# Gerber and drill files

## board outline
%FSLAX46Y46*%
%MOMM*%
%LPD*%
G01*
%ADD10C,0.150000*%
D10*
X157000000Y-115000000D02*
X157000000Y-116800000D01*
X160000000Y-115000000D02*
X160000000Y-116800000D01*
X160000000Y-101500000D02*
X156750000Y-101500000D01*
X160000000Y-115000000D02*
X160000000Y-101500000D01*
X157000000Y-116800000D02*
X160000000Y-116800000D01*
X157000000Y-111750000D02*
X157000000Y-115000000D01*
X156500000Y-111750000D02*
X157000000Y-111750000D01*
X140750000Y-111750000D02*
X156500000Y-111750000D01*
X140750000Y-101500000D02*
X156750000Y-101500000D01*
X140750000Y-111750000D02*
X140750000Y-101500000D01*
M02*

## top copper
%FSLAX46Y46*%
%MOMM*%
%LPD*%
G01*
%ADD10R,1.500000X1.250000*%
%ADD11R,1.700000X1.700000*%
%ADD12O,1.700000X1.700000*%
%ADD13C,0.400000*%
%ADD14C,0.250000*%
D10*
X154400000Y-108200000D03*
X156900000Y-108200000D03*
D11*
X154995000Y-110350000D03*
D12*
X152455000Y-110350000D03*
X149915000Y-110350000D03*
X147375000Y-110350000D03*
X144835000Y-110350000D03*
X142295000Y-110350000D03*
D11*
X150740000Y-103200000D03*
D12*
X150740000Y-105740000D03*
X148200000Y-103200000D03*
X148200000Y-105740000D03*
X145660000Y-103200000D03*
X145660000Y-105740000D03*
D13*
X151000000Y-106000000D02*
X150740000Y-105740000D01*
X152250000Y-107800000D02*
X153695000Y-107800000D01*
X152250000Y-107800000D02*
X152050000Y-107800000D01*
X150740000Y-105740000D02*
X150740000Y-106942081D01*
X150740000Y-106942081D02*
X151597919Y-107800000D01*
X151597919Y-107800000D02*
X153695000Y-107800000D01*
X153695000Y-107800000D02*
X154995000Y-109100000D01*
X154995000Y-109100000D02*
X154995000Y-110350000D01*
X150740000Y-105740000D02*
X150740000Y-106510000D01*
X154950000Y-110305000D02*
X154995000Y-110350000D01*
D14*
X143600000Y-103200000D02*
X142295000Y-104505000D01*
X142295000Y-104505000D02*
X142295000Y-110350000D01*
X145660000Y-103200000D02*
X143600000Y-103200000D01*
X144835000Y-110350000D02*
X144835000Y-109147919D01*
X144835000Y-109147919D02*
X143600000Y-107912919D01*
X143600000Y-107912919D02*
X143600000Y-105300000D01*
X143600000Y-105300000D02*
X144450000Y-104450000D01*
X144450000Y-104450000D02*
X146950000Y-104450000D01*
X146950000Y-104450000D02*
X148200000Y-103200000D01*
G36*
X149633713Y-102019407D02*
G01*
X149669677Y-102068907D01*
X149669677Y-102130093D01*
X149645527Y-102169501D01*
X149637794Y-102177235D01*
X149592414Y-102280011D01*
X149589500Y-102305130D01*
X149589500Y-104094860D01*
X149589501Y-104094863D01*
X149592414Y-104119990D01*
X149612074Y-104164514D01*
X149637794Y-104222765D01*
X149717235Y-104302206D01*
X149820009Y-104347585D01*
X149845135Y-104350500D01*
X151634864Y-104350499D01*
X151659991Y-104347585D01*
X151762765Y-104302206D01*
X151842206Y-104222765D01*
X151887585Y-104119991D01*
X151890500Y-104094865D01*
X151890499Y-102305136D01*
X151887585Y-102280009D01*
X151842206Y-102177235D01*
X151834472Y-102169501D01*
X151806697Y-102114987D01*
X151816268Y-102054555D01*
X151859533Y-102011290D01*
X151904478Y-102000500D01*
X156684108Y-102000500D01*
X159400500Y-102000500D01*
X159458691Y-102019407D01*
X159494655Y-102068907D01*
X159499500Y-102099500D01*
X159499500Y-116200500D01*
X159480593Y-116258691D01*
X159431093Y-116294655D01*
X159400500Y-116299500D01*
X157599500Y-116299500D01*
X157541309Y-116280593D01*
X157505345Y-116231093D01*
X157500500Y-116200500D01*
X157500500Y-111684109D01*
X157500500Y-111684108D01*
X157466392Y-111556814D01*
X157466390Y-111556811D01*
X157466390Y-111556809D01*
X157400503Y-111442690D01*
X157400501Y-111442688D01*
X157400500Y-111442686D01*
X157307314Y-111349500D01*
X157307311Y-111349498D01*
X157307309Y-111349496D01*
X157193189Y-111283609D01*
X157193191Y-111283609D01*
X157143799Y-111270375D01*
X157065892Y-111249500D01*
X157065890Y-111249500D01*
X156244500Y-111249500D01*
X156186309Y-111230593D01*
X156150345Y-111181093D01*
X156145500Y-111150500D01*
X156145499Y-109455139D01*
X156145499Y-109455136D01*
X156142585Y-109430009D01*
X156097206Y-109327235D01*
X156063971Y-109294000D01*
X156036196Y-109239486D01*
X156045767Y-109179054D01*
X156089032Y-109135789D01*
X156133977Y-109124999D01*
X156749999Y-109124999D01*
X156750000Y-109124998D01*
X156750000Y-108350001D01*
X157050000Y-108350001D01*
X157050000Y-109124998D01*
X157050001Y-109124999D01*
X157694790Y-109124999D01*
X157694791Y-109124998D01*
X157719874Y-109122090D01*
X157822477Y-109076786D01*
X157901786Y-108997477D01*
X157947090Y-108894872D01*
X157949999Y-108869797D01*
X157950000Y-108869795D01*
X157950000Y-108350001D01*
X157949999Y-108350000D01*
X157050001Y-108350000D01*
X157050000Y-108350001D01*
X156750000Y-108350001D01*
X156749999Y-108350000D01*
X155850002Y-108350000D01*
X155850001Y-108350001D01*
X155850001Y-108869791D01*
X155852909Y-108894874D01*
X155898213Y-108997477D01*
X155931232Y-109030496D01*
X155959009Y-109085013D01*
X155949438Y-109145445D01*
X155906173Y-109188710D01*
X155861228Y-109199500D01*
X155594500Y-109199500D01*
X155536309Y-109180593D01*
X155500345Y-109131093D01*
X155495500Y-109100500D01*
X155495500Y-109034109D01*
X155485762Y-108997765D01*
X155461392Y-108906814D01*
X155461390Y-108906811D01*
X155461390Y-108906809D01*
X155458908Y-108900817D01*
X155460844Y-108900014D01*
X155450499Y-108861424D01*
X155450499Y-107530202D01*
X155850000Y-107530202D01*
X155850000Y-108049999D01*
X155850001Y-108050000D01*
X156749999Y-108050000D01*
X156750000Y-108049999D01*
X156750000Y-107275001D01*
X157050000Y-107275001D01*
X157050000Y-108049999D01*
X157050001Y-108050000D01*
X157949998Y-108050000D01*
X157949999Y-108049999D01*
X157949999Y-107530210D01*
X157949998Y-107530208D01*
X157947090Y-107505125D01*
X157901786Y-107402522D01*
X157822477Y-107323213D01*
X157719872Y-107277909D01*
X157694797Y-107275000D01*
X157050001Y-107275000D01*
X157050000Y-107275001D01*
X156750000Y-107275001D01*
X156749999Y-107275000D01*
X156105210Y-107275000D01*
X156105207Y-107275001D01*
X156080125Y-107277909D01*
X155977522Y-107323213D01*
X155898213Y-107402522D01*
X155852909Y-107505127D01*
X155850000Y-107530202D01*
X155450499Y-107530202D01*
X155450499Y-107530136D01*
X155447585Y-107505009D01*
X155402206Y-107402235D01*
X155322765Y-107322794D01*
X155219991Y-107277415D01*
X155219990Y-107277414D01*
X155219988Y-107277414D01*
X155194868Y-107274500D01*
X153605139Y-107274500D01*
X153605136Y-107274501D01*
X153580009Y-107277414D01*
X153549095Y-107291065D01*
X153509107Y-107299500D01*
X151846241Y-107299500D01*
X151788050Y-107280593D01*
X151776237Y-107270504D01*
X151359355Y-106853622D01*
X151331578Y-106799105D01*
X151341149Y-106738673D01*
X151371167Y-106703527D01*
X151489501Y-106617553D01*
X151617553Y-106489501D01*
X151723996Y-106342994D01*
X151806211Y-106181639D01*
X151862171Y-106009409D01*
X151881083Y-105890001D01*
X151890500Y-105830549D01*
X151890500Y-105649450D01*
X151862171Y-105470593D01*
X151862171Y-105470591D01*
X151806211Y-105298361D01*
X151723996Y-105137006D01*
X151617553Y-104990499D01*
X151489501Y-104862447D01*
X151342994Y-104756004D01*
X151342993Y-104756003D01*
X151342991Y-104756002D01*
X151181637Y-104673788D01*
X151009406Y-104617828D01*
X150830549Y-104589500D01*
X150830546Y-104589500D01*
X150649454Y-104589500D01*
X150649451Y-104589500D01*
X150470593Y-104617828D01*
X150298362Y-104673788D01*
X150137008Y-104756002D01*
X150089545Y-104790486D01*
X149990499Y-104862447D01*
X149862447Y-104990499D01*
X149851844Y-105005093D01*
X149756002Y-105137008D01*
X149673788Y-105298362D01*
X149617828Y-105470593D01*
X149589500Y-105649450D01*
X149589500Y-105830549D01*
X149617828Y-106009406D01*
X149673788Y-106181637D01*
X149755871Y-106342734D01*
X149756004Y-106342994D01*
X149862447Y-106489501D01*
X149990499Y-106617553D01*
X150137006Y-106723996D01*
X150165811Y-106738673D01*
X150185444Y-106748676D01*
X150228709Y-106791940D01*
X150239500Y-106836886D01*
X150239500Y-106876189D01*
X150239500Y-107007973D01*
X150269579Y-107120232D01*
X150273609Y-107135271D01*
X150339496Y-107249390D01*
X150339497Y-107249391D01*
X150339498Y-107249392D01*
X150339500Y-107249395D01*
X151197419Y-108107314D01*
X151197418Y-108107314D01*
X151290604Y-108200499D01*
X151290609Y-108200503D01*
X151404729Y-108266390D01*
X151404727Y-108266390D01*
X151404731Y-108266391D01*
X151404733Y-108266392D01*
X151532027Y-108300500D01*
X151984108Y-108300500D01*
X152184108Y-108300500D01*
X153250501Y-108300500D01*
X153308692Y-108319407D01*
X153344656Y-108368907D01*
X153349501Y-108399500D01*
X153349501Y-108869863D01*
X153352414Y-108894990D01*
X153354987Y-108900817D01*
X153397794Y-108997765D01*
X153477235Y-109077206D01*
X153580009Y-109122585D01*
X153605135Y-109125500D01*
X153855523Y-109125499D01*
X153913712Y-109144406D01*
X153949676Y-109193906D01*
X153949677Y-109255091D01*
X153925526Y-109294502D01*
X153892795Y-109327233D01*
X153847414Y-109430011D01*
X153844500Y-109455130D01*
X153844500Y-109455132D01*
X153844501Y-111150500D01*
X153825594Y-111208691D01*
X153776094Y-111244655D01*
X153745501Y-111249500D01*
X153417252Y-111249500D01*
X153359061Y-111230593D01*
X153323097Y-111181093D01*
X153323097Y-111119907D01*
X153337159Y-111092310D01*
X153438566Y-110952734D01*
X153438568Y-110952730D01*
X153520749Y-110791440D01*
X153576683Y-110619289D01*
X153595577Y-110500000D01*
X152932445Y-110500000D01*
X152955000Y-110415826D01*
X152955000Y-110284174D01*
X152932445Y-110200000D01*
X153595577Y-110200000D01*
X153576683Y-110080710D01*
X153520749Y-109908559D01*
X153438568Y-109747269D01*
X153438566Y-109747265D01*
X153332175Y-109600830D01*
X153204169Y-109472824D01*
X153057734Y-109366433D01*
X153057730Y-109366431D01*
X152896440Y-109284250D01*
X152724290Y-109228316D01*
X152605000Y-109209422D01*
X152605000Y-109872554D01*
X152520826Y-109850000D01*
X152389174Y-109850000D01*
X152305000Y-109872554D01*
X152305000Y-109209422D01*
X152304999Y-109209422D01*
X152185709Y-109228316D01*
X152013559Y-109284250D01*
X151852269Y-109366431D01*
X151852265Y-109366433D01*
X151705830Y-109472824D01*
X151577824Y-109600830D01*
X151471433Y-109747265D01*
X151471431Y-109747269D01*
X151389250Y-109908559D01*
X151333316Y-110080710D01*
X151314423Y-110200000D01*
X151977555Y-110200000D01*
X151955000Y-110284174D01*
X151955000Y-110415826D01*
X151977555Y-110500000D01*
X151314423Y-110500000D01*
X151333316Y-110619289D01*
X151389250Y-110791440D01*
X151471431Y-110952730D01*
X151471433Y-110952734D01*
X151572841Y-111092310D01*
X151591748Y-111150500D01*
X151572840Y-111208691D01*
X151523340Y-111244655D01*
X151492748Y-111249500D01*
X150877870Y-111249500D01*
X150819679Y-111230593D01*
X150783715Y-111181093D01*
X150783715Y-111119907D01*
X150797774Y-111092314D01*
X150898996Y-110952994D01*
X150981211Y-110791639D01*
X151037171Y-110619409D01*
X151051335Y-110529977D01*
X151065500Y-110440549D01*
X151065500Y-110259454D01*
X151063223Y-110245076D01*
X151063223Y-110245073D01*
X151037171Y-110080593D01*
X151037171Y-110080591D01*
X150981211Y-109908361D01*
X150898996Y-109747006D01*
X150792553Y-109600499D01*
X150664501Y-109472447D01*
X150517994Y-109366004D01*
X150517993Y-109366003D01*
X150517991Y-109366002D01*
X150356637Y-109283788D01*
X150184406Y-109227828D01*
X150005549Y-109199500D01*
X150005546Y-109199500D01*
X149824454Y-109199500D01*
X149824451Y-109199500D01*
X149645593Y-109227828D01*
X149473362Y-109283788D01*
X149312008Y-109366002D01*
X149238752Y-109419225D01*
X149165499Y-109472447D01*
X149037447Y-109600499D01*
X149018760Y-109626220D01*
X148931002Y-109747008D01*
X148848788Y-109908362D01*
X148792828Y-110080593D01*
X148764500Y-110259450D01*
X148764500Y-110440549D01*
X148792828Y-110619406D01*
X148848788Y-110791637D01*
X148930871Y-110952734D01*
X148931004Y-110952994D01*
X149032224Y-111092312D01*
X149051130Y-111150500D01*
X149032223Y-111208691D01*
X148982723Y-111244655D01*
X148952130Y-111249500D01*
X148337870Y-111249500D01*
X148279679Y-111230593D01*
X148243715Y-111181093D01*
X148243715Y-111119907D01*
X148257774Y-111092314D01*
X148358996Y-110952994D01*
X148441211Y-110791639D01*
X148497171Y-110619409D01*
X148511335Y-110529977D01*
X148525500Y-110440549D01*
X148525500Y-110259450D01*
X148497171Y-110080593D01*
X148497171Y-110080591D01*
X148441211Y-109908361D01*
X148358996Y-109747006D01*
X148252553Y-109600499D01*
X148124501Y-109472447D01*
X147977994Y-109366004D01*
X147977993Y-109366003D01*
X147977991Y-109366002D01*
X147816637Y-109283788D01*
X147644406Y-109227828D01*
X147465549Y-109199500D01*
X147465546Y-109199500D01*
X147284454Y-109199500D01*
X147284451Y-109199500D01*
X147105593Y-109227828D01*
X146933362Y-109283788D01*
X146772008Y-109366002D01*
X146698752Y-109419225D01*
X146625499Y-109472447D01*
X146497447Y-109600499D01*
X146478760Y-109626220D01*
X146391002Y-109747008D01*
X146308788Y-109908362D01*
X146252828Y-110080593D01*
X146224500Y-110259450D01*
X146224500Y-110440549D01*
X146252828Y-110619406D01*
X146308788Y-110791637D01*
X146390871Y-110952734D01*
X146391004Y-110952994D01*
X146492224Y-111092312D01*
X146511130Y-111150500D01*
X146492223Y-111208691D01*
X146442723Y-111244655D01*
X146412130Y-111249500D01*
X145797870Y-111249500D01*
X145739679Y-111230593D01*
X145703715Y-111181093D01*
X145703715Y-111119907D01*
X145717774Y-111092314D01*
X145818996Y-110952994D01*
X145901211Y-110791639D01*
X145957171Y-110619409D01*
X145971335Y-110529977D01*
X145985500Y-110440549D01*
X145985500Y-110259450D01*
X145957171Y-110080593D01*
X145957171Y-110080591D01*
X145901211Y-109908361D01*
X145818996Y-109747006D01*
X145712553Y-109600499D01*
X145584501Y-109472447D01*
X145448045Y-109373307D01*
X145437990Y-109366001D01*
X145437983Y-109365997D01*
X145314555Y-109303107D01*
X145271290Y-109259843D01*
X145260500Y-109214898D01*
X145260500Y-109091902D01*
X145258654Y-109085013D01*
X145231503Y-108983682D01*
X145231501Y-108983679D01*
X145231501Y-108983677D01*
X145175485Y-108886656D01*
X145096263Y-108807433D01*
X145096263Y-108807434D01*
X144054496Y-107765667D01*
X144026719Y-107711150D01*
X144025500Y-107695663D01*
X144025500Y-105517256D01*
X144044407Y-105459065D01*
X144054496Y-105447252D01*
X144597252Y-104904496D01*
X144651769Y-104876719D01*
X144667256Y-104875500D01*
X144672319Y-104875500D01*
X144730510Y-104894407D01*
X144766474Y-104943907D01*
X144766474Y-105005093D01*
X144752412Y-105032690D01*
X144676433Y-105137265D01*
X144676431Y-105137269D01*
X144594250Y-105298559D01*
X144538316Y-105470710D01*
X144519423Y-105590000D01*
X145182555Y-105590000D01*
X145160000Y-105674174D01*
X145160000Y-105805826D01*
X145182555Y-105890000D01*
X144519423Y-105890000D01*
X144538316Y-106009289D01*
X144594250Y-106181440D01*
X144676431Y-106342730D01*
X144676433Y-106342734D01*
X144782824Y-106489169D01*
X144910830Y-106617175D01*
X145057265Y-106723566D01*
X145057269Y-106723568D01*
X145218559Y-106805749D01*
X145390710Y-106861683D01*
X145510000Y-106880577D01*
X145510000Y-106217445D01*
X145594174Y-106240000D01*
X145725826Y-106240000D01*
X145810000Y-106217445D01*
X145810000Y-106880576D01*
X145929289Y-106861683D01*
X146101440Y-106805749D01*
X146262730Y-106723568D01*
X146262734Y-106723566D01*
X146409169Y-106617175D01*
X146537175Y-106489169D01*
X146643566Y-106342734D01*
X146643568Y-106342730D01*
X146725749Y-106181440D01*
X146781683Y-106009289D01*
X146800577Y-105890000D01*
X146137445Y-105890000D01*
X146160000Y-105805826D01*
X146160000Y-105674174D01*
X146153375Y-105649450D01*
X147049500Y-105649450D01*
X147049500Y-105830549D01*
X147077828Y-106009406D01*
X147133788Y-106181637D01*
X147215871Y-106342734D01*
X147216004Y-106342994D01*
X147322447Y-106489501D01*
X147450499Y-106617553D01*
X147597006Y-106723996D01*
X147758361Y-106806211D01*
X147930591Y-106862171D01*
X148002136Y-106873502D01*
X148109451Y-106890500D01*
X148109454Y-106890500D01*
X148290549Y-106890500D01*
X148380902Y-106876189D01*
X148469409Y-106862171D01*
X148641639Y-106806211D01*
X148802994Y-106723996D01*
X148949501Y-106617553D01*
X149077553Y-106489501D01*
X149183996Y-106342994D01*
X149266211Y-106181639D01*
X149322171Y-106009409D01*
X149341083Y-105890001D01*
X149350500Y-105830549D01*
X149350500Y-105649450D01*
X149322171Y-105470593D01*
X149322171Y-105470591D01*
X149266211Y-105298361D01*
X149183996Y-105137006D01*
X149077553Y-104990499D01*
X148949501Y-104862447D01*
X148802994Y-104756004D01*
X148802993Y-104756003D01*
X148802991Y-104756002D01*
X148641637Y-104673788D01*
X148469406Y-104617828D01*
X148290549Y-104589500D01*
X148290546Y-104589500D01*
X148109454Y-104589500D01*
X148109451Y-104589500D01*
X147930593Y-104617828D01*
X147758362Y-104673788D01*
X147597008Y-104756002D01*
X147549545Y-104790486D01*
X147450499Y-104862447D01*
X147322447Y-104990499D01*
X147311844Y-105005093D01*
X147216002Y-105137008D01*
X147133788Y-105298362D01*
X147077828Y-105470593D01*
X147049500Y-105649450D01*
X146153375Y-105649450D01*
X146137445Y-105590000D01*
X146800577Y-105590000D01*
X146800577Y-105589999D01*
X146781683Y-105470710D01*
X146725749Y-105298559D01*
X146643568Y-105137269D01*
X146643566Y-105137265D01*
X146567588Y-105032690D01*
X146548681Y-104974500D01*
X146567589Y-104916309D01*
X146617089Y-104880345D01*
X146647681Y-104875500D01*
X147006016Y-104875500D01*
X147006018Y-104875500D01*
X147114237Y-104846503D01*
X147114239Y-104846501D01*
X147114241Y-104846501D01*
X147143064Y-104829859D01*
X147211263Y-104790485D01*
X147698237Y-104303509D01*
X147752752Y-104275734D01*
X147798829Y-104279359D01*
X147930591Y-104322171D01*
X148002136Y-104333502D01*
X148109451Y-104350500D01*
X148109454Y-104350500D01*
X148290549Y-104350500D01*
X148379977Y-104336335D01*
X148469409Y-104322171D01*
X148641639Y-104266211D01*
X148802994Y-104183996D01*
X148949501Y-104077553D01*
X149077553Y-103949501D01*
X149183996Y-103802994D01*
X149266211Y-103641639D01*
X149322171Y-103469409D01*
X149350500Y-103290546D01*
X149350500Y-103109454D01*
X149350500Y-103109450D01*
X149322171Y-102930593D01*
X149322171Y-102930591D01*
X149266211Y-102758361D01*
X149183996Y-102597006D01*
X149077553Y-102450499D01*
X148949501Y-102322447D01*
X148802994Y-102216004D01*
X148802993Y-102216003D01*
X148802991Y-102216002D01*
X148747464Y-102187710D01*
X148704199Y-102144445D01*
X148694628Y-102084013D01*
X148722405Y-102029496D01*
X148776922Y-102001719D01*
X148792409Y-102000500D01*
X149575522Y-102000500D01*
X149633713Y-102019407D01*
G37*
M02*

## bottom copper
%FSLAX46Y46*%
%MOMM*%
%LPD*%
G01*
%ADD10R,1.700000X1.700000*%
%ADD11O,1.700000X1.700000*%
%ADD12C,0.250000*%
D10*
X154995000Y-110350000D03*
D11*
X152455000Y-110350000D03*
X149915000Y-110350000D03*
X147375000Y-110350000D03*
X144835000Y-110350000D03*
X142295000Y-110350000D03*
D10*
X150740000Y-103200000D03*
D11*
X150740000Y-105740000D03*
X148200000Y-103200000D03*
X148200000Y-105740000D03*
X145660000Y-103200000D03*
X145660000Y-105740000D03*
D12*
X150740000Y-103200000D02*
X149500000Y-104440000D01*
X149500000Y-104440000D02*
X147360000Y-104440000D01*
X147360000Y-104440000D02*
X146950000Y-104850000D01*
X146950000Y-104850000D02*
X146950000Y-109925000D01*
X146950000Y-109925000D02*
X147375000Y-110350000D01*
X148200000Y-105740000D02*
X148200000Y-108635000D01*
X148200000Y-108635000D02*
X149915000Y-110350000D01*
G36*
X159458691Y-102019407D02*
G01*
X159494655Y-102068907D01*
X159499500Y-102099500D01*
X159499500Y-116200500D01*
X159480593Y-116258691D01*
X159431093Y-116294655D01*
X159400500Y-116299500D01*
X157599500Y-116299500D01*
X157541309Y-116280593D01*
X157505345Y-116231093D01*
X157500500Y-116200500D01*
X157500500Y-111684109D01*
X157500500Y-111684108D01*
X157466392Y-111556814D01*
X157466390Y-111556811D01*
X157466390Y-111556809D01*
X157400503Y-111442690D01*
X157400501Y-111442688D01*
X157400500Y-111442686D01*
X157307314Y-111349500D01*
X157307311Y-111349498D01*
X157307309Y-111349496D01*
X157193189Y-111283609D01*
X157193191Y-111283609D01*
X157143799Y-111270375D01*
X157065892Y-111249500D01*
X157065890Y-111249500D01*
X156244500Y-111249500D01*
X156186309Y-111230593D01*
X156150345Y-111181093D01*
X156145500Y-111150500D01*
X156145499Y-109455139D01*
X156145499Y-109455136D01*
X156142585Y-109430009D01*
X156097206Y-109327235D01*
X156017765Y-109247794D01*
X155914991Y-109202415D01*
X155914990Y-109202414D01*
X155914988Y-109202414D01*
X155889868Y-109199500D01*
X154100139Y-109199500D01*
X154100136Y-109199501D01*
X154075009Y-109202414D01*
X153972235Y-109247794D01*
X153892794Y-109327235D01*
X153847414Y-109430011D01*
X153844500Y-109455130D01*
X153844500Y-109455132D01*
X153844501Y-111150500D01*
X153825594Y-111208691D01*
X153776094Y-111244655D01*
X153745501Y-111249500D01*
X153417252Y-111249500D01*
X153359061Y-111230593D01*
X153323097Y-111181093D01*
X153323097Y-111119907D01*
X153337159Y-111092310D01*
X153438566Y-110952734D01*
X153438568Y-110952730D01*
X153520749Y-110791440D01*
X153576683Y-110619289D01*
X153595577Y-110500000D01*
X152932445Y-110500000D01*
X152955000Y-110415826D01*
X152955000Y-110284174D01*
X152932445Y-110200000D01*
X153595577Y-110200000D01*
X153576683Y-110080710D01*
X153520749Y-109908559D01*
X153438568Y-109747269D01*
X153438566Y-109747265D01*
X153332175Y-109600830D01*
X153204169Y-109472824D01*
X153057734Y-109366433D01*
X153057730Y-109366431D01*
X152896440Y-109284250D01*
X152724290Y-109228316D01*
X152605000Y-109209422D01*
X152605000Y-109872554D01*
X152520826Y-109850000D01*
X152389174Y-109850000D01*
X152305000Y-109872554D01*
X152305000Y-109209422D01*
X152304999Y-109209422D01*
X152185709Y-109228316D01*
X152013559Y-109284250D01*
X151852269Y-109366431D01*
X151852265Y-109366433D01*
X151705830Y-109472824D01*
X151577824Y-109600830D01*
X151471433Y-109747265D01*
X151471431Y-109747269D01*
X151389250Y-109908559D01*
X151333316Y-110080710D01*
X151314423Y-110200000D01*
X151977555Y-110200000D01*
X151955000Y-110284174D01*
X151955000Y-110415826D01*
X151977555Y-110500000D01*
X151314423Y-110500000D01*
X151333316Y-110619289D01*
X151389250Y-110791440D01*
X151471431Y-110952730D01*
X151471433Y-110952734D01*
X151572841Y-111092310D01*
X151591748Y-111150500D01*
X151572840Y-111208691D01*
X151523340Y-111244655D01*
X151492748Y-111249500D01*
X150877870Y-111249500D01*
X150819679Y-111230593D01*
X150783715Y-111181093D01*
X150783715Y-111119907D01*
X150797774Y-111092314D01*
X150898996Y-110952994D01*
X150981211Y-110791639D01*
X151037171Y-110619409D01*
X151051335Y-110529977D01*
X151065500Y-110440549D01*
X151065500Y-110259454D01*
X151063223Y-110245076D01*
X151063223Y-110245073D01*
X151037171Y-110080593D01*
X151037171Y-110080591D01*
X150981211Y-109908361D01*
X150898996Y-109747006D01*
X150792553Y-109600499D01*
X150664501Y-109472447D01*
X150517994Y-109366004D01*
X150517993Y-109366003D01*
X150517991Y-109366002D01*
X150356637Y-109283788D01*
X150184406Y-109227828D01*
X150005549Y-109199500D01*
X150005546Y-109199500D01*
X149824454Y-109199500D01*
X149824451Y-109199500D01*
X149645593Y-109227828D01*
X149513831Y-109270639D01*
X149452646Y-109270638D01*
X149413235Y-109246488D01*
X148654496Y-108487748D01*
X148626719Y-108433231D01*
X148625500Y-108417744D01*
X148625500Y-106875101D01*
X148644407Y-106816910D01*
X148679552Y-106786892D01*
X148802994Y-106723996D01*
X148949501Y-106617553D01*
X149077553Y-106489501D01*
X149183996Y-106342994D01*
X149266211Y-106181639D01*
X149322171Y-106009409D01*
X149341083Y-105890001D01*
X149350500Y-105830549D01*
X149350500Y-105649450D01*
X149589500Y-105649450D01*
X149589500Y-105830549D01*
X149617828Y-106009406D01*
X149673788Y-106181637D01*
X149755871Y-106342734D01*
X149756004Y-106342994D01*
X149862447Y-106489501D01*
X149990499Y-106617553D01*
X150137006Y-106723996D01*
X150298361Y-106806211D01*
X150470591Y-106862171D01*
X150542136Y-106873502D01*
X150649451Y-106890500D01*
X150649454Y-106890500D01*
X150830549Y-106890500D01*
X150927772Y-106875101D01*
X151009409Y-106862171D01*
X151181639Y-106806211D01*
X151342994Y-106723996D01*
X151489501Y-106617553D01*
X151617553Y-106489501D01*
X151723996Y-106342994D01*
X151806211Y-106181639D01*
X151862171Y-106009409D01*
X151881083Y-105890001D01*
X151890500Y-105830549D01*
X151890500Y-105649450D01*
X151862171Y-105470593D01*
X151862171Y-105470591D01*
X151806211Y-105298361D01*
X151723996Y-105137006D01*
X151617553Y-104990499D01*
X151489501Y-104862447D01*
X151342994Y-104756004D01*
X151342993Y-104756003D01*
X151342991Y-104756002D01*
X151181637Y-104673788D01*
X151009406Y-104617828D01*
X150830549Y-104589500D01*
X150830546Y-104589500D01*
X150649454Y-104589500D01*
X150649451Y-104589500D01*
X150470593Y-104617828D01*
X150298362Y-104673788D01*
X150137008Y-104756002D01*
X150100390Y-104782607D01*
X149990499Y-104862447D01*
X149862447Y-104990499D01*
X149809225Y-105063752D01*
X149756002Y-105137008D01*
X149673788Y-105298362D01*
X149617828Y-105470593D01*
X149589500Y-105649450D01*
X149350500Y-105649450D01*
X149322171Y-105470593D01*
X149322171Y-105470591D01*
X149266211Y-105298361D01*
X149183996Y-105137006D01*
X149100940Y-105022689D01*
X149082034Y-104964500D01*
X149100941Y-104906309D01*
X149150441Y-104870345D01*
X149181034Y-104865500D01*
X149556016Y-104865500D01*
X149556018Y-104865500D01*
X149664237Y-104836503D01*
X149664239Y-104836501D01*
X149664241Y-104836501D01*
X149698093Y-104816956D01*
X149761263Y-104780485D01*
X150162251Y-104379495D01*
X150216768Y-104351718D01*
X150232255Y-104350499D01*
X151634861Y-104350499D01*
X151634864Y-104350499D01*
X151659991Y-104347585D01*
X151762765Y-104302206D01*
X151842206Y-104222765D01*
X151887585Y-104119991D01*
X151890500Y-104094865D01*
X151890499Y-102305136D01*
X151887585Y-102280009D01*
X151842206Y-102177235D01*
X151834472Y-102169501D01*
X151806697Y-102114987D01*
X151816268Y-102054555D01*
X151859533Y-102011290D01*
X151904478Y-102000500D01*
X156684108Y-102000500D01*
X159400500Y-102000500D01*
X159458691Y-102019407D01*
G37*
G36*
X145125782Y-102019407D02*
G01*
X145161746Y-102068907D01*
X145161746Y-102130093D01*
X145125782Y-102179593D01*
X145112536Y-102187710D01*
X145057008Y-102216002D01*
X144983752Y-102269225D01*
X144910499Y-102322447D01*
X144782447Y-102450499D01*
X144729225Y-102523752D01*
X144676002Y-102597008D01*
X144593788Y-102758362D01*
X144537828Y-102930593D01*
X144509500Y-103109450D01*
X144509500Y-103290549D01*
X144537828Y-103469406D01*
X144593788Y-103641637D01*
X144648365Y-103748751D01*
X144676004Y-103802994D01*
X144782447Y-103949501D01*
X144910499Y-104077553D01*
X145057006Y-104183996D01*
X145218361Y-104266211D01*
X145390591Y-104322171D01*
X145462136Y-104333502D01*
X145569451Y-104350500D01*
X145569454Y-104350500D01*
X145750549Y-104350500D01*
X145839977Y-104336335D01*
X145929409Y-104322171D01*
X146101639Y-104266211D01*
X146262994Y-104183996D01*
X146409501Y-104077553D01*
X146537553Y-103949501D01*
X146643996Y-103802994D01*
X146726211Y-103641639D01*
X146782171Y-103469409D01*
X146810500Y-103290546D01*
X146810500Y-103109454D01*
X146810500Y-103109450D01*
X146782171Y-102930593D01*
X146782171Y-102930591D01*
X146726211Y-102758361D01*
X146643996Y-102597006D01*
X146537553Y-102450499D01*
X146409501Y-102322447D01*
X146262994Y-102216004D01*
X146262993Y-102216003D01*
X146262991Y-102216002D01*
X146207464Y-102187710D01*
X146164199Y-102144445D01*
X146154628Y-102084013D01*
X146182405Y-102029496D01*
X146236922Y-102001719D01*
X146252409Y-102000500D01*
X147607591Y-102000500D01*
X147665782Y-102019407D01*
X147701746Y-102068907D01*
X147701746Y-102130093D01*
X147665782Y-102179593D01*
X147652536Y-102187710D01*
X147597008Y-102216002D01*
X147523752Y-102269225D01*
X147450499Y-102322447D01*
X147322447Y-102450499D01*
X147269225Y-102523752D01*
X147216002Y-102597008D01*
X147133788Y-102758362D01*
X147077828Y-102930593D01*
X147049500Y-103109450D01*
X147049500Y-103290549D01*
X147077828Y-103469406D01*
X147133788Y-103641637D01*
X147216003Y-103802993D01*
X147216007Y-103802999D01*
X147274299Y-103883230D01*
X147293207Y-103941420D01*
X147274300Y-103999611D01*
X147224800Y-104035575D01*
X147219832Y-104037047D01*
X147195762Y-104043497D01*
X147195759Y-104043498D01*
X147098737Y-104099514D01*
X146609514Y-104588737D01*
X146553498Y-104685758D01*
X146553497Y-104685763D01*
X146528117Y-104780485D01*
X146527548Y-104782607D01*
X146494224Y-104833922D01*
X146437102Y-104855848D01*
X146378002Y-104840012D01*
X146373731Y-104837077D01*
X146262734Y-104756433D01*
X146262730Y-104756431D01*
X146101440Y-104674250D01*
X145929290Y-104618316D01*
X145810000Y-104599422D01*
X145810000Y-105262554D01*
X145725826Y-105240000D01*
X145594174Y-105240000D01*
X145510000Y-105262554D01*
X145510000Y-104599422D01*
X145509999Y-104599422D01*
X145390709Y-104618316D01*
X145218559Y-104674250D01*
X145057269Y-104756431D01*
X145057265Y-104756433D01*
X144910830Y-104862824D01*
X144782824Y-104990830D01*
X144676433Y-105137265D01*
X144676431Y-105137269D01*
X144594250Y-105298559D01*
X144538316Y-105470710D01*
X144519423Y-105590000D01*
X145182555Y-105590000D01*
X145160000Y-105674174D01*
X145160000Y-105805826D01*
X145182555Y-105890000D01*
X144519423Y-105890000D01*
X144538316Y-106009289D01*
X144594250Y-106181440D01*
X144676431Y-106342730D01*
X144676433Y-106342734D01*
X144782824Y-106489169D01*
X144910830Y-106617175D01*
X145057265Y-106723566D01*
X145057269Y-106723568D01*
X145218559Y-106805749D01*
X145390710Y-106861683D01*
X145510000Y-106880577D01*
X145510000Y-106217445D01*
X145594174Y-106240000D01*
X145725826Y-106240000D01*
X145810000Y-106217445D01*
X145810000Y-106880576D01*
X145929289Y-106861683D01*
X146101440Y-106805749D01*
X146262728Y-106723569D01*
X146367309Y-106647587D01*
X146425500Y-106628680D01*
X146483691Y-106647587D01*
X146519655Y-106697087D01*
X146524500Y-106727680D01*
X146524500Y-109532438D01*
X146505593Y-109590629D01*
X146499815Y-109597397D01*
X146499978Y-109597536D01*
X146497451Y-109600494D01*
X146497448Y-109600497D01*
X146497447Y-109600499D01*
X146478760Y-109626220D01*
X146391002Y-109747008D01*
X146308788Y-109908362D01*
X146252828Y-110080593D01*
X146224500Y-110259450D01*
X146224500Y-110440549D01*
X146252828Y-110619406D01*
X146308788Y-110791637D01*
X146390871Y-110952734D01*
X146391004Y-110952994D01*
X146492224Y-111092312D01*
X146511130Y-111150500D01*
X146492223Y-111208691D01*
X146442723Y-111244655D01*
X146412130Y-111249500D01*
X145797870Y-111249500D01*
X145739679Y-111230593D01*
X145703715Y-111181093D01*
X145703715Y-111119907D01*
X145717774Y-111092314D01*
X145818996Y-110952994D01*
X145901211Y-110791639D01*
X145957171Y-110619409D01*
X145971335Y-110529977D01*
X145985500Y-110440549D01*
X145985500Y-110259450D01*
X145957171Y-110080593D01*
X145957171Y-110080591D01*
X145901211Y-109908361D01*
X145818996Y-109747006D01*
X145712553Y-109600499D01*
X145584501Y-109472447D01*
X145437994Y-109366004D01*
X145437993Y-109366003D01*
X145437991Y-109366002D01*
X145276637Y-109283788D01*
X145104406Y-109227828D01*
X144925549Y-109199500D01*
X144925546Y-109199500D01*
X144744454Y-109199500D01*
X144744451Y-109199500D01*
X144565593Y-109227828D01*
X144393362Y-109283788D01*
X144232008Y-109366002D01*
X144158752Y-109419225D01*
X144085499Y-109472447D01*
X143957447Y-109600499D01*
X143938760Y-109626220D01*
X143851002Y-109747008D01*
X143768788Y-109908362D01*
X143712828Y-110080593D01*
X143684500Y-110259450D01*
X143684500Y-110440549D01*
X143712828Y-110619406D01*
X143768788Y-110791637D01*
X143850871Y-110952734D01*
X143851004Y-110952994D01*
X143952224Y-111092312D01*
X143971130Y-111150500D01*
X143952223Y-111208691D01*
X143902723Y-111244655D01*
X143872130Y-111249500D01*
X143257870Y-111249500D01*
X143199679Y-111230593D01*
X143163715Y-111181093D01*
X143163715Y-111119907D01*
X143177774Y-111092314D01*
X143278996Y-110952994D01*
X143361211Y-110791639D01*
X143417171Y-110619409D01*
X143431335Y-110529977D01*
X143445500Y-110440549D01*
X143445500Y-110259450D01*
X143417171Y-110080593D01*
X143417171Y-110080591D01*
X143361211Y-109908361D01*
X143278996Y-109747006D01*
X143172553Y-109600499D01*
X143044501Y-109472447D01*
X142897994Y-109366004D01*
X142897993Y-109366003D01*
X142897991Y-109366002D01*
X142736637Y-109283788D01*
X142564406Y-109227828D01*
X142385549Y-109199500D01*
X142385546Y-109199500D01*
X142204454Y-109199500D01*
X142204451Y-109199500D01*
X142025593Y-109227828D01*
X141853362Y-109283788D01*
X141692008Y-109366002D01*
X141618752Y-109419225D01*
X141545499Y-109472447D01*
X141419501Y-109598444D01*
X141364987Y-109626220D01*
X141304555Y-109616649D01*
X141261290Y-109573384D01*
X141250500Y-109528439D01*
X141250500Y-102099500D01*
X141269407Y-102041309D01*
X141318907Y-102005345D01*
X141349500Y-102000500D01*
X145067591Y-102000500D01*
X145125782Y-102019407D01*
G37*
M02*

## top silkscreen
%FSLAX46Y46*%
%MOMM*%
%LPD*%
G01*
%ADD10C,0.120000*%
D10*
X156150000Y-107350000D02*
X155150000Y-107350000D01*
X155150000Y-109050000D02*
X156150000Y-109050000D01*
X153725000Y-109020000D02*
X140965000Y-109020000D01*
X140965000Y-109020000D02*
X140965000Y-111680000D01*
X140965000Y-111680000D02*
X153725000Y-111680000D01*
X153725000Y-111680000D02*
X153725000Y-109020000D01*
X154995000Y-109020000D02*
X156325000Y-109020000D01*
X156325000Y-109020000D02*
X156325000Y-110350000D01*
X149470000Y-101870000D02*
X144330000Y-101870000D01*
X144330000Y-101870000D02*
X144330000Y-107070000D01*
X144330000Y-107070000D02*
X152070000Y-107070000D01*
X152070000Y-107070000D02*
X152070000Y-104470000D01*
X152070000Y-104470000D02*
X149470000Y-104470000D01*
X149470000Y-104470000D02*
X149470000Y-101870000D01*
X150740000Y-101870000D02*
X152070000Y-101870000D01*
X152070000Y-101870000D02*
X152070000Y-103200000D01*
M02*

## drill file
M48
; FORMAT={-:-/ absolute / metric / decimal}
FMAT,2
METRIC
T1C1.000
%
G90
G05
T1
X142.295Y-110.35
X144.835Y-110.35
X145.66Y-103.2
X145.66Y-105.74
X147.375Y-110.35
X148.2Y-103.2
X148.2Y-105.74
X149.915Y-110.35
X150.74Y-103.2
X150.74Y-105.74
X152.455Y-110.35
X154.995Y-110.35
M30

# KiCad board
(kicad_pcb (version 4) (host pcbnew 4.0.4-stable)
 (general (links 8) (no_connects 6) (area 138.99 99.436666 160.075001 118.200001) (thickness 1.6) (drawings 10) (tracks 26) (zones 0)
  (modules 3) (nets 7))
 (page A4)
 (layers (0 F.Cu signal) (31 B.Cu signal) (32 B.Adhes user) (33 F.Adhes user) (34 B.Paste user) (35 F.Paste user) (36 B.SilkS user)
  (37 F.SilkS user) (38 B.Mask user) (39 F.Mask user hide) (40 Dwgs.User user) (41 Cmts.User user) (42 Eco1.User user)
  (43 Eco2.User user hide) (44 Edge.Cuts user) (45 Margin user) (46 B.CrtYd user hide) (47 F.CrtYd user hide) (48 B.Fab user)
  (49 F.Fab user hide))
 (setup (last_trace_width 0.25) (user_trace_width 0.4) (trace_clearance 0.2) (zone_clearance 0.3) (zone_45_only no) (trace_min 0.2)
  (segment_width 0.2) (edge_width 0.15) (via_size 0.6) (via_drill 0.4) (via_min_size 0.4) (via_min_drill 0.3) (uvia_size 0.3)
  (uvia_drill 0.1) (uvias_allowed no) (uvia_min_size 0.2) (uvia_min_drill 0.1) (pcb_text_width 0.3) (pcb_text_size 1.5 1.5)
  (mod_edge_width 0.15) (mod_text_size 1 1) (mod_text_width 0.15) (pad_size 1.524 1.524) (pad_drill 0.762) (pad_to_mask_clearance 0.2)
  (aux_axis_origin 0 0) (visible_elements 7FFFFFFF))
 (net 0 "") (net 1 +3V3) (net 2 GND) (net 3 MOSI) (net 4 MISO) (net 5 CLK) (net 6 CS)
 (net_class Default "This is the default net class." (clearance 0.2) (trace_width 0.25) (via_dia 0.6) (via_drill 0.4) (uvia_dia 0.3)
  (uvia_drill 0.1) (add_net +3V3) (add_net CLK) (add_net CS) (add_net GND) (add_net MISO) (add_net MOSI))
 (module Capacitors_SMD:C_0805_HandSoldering (layer F.Cu) (at 155.65 108.2)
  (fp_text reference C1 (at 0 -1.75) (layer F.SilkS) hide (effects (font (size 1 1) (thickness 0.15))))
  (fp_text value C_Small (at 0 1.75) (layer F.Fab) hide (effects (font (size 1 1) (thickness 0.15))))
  (fp_line (start 0.5 -0.85) (end -0.5 -0.85) (layer F.SilkS) (width 0.12))
  (fp_line (start -0.5 0.85) (end 0.5 0.85) (layer F.SilkS) (width 0.12))
  (pad 1 smd rect (at -1.25 0) (size 1.5 1.25) (layers F.Cu F.Paste F.Mask) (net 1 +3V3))
  (pad 2 smd rect (at 1.25 0) (size 1.5 1.25) (layers F.Cu F.Paste F.Mask) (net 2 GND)))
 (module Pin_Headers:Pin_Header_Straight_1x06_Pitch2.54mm (layer F.Cu) (at 154.995 110.35 270)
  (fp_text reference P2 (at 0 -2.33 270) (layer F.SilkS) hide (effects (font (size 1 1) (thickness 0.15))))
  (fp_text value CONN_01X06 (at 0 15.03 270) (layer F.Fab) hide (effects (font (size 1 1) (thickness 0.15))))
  (fp_line (start -1.33 1.27) (end -1.33 14.03) (layer F.SilkS) (width 0.12))
  (fp_line (start -1.33 14.03) (end 1.33 14.03) (layer F.SilkS) (width 0.12))
  (fp_line (start 1.33 14.03) (end 1.33 1.27) (layer F.SilkS) (width 0.12))
  (fp_line (start 1.33 1.27) (end -1.33 1.27) (layer F.SilkS) (width 0.12))
  (fp_line (start -1.33 0) (end -1.33 -1.33) (layer F.SilkS) (width 0.12))
  (fp_line (start -1.33 -1.33) (end 0 -1.33) (layer F.SilkS) (width 0.12))
  (pad 1 thru_hole rect (at 0 0 270) (size 1.7 1.7) (drill 1) (layers *.Cu *.Mask) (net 1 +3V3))
  (pad 2 thru_hole oval (at 0 2.54 270) (size 1.7 1.7) (drill 1) (layers *.Cu *.Mask) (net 2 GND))
  (pad 3 thru_hole oval (at 0 5.08 270) (size 1.7 1.7) (drill 1) (layers *.Cu *.Mask) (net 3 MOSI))
  (pad 4 thru_hole oval (at 0 7.62 270) (size 1.7 1.7) (drill 1) (layers *.Cu *.Mask) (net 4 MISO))
  (pad 5 thru_hole oval (at 0 10.16 270) (size 1.7 1.7) (drill 1) (layers *.Cu *.Mask) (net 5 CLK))
  (pad 6 thru_hole oval (at 0 12.7 270) (size 1.7 1.7) (drill 1) (layers *.Cu *.Mask) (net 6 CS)))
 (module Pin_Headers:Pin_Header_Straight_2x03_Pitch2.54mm (layer F.Cu) (at 150.74 103.2 270)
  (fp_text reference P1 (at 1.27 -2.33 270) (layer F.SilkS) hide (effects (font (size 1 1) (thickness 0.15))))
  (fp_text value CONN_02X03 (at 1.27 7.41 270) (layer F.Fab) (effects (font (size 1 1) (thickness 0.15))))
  (fp_line (start -1.33 1.27) (end -1.33 6.41) (layer F.SilkS) (width 0.12))
  (fp_line (start -1.33 6.41) (end 3.87 6.41) (layer F.SilkS) (width 0.12))
  (fp_line (start 3.87 6.41) (end 3.87 -1.33) (layer F.SilkS) (width 0.12))
  (fp_line (start 3.87 -1.33) (end 1.27 -1.33) (layer F.SilkS) (width 0.12))
  (fp_line (start 1.27 -1.33) (end 1.27 1.27) (layer F.SilkS) (width 0.12))
  (fp_line (start 1.27 1.27) (end -1.33 1.27) (layer F.SilkS) (width 0.12))
  (fp_line (start -1.33 0) (end -1.33 -1.33) (layer F.SilkS) (width 0.12))
  (fp_line (start -1.33 -1.33) (end 0 -1.33) (layer F.SilkS) (width 0.12))
  (pad 1 thru_hole rect (at 0 0 270) (size 1.7 1.7) (drill 1) (layers *.Cu *.Mask) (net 4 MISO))
  (pad 2 thru_hole oval (at 2.54 0 270) (size 1.7 1.7) (drill 1) (layers *.Cu *.Mask) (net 1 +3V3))
  (pad 3 thru_hole oval (at 0 2.54 270) (size 1.7 1.7) (drill 1) (layers *.Cu *.Mask) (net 5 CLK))
  (pad 4 thru_hole oval (at 2.54 2.54 270) (size 1.7 1.7) (drill 1) (layers *.Cu *.Mask) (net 3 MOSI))
  (pad 5 thru_hole oval (at 0 5.08 270) (size 1.7 1.7) (drill 1) (layers *.Cu *.Mask) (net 6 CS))
  (pad 6 thru_hole oval (at 2.54 5.08 270) (size 1.7 1.7) (drill 1) (layers *.Cu *.Mask) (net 2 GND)))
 (gr_line (start 157 115) (end 157 116.8) (layer Edge.Cuts) (width 0.15))
 (gr_line (start 160 115) (end 160 116.8) (layer Edge.Cuts) (width 0.15))
 (gr_line (start 160 101.5) (end 156.75 101.5) (layer Edge.Cuts) (width 0.15))
 (gr_line (start 160 115) (end 160 101.5) (layer Edge.Cuts) (width 0.15))
 (gr_line (start 157 116.8) (end 160 116.8) (layer Edge.Cuts) (width 0.15))
 (gr_line (start 157 111.75) (end 157 115) (layer Edge.Cuts) (width 0.15))
 (gr_line (start 156.5 111.75) (end 157 111.75) (layer Edge.Cuts) (width 0.15))
 (gr_line (start 140.75 111.75) (end 156.5 111.75) (layer Edge.Cuts) (width 0.15))
 (gr_line (start 140.75 101.5) (end 156.75 101.5) (layer Edge.Cuts) (width 0.15))
 (gr_line (start 140.75 111.75) (end 140.75 101.5) (layer Edge.Cuts) (width 0.15))
 (segment (start 151 106) (end 150.74 105.74) (width 0.4) (layer F.Cu) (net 1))
 (segment (start 152.25 107.8) (end 153.695 107.8) (width 0.4) (layer F.Cu) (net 1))
 (segment (start 152.25 107.8) (end 152.05 107.8) (width 0.4) (layer F.Cu) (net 1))
 (segment (start 150.74 105.74) (end 150.74 106.942081) (width 0.4) (layer F.Cu) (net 1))
 (segment (start 150.74 106.942081) (end 151.597919 107.8) (width 0.4) (layer F.Cu) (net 1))
 (segment (start 151.597919 107.8) (end 153.695 107.8) (width 0.4) (layer F.Cu) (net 1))
 (segment (start 153.695 107.8) (end 154.995 109.1) (width 0.4) (layer F.Cu) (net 1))
 (segment (start 154.995 109.1) (end 154.995 110.35) (width 0.4) (layer F.Cu) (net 1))
 (segment (start 150.74 105.74) (end 150.74 106.51) (width 0.4) (layer F.Cu) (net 1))
 (segment (start 154.95 110.305) (end 154.995 110.35) (width 0.4) (layer F.Cu) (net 1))
 (segment (start 143.6 103.2) (end 142.295 104.505) (width 0.25) (layer F.Cu) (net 6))
 (segment (start 142.295 104.505) (end 142.295 110.35) (width 0.25) (layer F.Cu) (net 6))
 (segment (start 145.66 103.2) (end 143.6 103.2) (width 0.25) (layer F.Cu) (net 6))
 (segment (start 150.74 103.2) (end 149.5 104.44) (width 0.25) (layer B.Cu) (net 4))
 (segment (start 149.5 104.44) (end 147.36 104.44) (width 0.25) (layer B.Cu) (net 4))
 (segment (start 147.36 104.44) (end 146.95 104.85) (width 0.25) (layer B.Cu) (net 4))
 (segment (start 146.95 104.85) (end 146.95 109.925) (width 0.25) (layer B.Cu) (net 4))
 (segment (start 146.95 109.925) (end 147.375 110.35) (width 0.25) (layer B.Cu) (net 4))
 (segment (start 144.835 110.35) (end 144.835 109.147919) (width 0.25) (layer F.Cu) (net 5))
 (segment (start 144.835 109.147919) (end 143.6 107.912919) (width 0.25) (layer F.Cu) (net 5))
 (segment (start 143.6 107.912919) (end 143.6 105.3) (width 0.25) (layer F.Cu) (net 5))
 (segment (start 143.6 105.3) (end 144.45 104.45) (width 0.25) (layer F.Cu) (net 5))
 (segment (start 144.45 104.45) (end 146.95 104.45) (width 0.25) (layer F.Cu) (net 5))
 (segment (start 146.95 104.45) (end 148.2 103.2) (width 0.25) (layer F.Cu) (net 5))
 (segment (start 148.2 105.74) (end 148.2 108.635) (width 0.25) (layer B.Cu) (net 3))
 (segment (start 148.2 108.635) (end 149.915 110.35) (width 0.25) (layer B.Cu) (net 3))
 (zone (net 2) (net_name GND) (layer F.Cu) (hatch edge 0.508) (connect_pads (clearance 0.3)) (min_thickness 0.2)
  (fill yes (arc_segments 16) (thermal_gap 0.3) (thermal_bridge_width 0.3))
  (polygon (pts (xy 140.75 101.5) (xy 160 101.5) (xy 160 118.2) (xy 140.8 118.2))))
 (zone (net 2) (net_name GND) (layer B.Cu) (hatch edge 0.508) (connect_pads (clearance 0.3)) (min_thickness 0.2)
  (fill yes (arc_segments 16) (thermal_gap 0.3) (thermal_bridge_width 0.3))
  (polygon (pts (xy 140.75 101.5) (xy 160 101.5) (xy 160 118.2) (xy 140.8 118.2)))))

